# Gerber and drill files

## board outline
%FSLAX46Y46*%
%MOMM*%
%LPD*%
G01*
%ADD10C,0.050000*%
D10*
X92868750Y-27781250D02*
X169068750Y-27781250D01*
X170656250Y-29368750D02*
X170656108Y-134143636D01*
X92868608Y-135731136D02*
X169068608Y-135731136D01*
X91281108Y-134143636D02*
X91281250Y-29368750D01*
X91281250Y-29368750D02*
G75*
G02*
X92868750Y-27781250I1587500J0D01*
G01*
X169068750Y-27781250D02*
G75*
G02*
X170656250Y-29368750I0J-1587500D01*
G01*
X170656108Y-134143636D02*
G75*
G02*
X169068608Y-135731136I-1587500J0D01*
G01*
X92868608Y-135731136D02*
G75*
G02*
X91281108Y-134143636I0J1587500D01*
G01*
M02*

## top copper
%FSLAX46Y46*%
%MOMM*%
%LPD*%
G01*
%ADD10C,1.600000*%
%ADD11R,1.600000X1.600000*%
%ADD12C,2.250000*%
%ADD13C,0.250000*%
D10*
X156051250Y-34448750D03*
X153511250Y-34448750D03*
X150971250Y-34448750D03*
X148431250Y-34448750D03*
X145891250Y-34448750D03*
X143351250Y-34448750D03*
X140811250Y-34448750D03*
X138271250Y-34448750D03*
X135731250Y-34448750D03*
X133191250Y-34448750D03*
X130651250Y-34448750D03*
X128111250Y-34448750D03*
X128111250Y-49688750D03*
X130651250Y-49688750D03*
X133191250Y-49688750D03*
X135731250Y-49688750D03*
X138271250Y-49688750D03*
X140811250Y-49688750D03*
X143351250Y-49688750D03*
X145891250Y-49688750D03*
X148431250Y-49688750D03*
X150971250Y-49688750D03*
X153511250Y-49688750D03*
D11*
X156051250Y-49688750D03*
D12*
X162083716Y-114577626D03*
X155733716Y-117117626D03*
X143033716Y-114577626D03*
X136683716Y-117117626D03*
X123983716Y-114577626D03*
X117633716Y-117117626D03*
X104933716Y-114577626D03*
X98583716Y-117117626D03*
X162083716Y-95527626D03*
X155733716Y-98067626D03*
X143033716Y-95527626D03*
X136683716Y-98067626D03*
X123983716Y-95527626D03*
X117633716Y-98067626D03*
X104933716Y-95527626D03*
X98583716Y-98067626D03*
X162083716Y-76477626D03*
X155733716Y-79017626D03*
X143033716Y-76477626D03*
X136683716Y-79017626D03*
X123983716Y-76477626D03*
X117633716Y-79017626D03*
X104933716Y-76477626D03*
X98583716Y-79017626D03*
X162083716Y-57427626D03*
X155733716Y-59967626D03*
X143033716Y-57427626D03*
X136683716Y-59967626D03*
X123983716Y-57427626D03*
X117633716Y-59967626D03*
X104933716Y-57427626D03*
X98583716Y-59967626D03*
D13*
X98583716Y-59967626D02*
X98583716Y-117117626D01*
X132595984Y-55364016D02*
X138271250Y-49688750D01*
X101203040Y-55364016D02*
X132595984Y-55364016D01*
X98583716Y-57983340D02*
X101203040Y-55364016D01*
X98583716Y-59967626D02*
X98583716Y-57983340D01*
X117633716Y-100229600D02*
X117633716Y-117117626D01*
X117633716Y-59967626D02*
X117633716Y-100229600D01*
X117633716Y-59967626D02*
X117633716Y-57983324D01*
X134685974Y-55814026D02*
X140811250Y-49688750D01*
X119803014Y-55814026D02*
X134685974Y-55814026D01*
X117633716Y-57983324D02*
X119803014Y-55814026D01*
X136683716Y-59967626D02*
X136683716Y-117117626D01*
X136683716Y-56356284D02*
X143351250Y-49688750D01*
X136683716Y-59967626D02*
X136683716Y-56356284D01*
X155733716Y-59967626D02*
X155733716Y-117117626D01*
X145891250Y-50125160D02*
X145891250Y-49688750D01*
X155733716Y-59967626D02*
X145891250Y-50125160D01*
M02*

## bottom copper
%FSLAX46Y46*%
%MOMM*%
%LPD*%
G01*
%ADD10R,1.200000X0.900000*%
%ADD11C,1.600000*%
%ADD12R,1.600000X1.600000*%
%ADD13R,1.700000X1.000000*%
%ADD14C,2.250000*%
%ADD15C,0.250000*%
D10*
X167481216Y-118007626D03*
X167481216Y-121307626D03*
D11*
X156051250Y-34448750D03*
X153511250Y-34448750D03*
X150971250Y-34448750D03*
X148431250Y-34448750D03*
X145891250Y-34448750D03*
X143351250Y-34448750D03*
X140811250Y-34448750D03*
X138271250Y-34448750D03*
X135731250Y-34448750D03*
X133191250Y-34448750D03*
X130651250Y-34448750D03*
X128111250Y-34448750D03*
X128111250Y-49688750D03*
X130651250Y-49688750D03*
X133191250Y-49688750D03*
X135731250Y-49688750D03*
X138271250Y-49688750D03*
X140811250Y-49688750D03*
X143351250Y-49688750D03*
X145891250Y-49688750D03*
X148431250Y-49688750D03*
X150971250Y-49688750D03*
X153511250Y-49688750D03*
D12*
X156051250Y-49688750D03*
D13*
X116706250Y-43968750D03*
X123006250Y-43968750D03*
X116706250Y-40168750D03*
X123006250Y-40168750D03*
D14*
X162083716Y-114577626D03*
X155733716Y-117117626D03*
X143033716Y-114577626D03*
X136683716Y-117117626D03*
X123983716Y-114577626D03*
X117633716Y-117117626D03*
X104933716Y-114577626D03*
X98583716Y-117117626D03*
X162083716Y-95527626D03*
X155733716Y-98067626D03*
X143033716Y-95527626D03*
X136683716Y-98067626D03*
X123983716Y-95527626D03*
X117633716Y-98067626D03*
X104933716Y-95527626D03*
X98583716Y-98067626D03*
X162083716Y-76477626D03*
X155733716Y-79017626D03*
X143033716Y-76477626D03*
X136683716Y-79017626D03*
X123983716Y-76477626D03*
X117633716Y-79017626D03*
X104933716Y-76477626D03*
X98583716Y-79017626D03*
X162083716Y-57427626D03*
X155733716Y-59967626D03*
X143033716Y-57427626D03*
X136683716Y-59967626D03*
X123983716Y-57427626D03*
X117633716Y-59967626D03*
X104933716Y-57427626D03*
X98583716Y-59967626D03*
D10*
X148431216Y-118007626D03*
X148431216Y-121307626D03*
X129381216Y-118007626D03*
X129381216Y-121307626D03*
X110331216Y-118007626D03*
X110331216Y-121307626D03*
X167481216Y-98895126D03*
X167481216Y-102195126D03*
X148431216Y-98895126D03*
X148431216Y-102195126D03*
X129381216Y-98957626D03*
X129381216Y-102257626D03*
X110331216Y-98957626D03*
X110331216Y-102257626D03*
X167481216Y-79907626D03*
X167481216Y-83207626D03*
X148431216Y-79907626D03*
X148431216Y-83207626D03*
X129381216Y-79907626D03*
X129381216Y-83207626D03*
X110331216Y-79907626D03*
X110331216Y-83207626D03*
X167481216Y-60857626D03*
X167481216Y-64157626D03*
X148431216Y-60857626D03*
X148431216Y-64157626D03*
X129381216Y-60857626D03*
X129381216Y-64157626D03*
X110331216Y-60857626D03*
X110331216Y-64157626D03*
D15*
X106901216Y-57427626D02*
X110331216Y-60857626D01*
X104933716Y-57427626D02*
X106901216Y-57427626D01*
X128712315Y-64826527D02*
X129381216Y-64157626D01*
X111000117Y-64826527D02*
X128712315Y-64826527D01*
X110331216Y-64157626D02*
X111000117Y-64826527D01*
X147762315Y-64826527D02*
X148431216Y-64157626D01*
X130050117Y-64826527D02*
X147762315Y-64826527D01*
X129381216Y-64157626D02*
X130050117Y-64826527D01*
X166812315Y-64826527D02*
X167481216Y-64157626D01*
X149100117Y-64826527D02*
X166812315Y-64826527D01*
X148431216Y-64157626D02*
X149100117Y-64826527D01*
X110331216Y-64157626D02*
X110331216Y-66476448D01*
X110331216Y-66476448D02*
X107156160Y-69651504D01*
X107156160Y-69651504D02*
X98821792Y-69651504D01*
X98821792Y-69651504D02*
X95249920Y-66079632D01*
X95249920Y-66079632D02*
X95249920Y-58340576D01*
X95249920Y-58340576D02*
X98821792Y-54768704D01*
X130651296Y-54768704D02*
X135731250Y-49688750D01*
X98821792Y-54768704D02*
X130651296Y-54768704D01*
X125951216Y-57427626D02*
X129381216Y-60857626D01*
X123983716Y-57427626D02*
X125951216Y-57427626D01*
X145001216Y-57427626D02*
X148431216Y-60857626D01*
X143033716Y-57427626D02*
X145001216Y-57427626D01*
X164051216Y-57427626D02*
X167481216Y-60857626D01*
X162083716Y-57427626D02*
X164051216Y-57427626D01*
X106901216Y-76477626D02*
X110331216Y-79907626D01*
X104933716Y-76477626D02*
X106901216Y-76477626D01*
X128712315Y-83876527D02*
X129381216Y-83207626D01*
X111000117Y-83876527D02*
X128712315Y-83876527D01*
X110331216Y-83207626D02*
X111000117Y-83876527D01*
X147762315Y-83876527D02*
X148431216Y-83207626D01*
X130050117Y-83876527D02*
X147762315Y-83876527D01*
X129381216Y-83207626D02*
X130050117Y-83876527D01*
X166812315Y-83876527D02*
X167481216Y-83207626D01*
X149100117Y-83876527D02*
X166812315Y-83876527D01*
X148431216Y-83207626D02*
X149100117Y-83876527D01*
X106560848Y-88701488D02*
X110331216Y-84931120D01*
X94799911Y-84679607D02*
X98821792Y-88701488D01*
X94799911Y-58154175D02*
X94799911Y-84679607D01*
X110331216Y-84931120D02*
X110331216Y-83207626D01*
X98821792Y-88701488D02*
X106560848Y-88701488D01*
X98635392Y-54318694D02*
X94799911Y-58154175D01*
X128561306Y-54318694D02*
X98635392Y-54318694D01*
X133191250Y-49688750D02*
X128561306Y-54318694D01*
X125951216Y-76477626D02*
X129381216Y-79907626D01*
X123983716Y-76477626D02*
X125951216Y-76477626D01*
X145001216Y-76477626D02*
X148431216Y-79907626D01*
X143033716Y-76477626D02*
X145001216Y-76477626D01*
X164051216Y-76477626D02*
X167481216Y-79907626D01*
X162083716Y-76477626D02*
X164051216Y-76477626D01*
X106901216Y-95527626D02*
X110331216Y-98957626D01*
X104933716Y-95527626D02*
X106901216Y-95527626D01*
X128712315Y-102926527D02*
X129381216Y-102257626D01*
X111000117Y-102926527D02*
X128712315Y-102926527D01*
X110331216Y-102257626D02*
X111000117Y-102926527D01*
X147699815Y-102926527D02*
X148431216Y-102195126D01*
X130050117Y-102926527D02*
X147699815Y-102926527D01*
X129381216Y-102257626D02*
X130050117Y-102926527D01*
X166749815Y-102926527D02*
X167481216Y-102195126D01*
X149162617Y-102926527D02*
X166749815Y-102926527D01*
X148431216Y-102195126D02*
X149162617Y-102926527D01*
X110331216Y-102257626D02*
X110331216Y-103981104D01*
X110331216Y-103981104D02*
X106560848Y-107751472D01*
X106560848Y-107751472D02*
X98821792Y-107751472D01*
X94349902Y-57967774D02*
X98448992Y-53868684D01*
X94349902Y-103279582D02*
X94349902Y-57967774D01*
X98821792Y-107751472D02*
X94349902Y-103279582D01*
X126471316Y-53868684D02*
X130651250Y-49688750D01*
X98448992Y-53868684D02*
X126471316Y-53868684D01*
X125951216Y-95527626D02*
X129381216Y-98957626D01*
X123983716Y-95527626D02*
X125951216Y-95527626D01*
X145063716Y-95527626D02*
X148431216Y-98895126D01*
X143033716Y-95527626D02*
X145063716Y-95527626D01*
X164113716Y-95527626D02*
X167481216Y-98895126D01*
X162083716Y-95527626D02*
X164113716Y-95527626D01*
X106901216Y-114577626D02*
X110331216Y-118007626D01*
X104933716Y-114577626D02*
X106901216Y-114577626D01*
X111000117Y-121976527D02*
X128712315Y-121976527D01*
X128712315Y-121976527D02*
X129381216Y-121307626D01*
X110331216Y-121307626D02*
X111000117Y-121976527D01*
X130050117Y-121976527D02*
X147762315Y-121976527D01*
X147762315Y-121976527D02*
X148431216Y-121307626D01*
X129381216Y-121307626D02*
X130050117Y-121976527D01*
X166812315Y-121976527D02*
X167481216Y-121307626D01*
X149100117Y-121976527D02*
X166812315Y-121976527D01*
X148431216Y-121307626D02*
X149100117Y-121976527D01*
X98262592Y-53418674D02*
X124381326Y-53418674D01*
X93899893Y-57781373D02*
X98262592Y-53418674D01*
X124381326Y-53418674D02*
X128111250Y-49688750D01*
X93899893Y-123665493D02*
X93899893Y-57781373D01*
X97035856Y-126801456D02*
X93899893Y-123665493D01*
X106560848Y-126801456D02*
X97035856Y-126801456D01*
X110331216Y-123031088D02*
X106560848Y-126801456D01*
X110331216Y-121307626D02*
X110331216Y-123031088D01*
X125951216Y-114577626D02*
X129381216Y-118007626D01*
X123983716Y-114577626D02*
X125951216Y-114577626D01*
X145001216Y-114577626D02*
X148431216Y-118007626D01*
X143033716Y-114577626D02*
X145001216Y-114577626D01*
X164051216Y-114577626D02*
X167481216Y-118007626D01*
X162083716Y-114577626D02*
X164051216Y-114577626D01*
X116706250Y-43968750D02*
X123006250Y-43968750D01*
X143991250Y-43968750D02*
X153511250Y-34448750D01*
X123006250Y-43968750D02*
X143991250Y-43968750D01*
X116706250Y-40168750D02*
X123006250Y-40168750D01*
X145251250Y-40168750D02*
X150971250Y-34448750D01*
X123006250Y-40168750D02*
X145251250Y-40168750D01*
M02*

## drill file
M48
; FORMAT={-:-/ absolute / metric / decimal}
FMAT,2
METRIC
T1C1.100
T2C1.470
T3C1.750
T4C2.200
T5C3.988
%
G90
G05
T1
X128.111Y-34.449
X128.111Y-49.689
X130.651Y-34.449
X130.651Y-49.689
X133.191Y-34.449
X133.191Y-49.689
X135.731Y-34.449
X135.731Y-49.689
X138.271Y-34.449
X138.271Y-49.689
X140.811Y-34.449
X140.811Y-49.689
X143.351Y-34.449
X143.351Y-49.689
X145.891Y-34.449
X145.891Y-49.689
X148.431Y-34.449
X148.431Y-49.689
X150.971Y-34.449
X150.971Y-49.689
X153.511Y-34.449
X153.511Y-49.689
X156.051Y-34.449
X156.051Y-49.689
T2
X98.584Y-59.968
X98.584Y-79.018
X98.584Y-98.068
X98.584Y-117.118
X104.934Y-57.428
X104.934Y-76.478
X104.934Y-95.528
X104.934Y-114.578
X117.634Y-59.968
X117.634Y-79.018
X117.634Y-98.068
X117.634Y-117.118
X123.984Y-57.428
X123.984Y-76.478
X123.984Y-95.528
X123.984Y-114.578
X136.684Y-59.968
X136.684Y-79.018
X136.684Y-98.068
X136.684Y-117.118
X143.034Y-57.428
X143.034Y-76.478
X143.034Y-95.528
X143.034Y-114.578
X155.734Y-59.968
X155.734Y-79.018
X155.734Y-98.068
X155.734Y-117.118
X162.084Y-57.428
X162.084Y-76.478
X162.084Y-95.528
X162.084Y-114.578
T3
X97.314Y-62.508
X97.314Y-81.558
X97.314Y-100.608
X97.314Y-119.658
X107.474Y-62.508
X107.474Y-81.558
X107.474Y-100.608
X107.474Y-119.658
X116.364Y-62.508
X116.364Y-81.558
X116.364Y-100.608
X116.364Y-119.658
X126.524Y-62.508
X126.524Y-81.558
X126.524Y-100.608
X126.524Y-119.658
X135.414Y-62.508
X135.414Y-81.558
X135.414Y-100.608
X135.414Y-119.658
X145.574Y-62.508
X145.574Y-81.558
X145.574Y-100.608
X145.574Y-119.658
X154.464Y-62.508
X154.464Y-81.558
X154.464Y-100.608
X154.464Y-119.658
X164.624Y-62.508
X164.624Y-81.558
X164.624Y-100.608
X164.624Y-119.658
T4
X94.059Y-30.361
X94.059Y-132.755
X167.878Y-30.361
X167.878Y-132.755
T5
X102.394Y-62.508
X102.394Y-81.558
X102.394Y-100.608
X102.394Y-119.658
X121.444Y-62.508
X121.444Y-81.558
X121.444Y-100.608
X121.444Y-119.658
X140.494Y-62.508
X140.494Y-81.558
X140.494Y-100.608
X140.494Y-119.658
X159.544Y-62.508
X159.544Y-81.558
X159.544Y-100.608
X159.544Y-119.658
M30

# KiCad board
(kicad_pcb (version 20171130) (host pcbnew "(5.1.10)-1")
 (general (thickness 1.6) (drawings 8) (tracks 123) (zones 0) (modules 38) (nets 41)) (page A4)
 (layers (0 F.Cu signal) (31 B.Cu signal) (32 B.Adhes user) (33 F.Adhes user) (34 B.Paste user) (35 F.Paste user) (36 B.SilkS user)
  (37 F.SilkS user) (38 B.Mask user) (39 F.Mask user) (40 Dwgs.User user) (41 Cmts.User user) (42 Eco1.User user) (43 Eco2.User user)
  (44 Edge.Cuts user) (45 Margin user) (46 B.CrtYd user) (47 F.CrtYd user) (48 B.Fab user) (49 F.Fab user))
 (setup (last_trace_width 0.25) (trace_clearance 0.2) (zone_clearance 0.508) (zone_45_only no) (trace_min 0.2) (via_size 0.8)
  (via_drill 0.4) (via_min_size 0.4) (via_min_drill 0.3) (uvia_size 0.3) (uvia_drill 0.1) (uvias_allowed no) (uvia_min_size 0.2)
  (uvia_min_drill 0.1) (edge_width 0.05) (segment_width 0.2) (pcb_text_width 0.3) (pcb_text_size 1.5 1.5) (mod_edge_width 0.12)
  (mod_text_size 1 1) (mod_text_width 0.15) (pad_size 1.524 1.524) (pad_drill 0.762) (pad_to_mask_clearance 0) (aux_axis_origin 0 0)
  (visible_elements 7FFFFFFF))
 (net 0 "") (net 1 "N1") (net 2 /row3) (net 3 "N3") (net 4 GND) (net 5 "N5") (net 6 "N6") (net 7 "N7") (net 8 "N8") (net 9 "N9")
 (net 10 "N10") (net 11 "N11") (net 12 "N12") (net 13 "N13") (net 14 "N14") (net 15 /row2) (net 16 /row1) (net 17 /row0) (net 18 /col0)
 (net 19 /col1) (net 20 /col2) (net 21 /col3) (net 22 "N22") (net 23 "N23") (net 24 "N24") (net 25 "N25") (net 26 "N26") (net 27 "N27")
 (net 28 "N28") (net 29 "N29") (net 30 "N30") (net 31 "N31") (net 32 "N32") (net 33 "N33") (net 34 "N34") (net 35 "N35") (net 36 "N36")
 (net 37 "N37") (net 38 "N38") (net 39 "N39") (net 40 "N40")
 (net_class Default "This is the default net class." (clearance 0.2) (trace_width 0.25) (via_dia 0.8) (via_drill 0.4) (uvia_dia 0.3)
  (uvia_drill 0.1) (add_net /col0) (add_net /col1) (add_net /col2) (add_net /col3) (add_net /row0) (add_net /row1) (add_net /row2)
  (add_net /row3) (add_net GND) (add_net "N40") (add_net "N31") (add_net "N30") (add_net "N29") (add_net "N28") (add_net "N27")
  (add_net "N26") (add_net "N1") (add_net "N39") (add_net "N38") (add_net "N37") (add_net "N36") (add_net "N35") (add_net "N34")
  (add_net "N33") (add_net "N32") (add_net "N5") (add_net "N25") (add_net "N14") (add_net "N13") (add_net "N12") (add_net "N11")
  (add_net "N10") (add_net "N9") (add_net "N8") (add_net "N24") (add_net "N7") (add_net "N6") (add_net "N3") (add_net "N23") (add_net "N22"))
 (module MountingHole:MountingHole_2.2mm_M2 (layer F.Cu) (at 167.877984 132.754576)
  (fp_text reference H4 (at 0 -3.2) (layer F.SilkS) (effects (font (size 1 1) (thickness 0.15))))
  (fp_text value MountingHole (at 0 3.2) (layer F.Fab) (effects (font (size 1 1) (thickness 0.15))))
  (pad 1 np_thru_hole circle (at 0 0) (size 2.2 2.2) (drill 2.2) (layers *.Cu *.Mask)))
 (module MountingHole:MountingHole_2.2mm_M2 (layer F.Cu) (at 94.059296 132.754576)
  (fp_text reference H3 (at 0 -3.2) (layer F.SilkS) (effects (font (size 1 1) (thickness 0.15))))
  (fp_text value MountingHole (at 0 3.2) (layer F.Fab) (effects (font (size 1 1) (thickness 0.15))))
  (pad 1 np_thru_hole circle (at 0 0) (size 2.2 2.2) (drill 2.2) (layers *.Cu *.Mask)))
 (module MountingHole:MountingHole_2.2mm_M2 (layer F.Cu) (at 167.877984 30.360912)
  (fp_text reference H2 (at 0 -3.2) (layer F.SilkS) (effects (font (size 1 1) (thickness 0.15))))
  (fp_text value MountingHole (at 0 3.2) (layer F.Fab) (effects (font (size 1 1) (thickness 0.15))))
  (pad 1 np_thru_hole circle (at 0 0) (size 2.2 2.2) (drill 2.2) (layers *.Cu *.Mask)))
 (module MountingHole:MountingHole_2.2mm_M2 (layer F.Cu) (at 94.059296 30.360912)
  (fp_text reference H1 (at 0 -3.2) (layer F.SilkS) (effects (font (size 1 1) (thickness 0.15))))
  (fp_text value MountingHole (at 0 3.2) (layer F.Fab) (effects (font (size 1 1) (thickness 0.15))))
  (pad 1 np_thru_hole circle (at 0 0) (size 2.2 2.2) (drill 2.2) (layers *.Cu *.Mask)))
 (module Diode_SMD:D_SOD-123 (layer B.Cu) (at 167.481216 119.657626 90)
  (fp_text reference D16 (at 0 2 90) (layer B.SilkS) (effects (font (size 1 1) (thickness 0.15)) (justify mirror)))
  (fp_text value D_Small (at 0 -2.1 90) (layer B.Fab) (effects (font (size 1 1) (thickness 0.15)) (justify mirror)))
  (pad 2 smd rect (at 1.65 0 90) (size 0.9 1.2) (layers B.Cu B.Paste B.Mask) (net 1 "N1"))
  (pad 1 smd rect (at -1.65 0 90) (size 0.9 1.2) (layers B.Cu B.Paste B.Mask) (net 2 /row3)))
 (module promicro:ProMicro (layer B.Cu) (at 142.08125 42.06875 180)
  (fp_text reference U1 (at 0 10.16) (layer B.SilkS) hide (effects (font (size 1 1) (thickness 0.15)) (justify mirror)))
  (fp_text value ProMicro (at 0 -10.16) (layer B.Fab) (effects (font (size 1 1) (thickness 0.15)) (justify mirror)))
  (pad 24 thru_hole circle (at -13.97 7.62 180) (size 1.6 1.6) (drill 1.1) (layers *.Cu *.Mask B.SilkS) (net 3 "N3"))
  (pad 23 thru_hole circle (at -11.43 7.62 180) (size 1.6 1.6) (drill 1.1) (layers *.Cu *.Mask B.SilkS) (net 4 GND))
  (pad 22 thru_hole circle (at -8.89 7.62 180) (size 1.6 1.6) (drill 1.1) (layers *.Cu *.Mask B.SilkS) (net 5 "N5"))
  (pad 21 thru_hole circle (at -6.35 7.62 180) (size 1.6 1.6) (drill 1.1) (layers *.Cu *.Mask B.SilkS) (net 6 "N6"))
  (pad 20 thru_hole circle (at -3.81 7.62 180) (size 1.6 1.6) (drill 1.1) (layers *.Cu *.Mask B.SilkS) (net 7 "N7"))
  (pad 19 thru_hole circle (at -1.27 7.62 180) (size 1.6 1.6) (drill 1.1) (layers *.Cu *.Mask B.SilkS) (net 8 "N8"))
  (pad 18 thru_hole circle (at 1.27 7.62 180) (size 1.6 1.6) (drill 1.1) (layers *.Cu *.Mask B.SilkS) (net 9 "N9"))
  (pad 17 thru_hole circle (at 3.81 7.62 180) (size 1.6 1.6) (drill 1.1) (layers *.Cu *.Mask B.SilkS) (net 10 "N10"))
  (pad 16 thru_hole circle (at 6.35 7.62 180) (size 1.6 1.6) (drill 1.1) (layers *.Cu *.Mask B.SilkS) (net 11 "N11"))
  (pad 15 thru_hole circle (at 8.89 7.62 180) (size 1.6 1.6) (drill 1.1) (layers *.Cu *.Mask B.SilkS) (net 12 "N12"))
  (pad 14 thru_hole circle (at 11.43 7.62 180) (size 1.6 1.6) (drill 1.1) (layers *.Cu *.Mask B.SilkS) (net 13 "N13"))
  (pad 13 thru_hole circle (at 13.97 7.62 180) (size 1.6 1.6) (drill 1.1) (layers *.Cu *.Mask B.SilkS) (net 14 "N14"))
  (pad 12 thru_hole circle (at 13.97 -7.62 180) (size 1.6 1.6) (drill 1.1) (layers *.Cu *.Mask B.SilkS) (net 2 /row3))
  (pad 11 thru_hole circle (at 11.43 -7.62 180) (size 1.6 1.6) (drill 1.1) (layers *.Cu *.Mask B.SilkS) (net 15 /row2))
  (pad 10 thru_hole circle (at 8.89 -7.62 180) (size 1.6 1.6) (drill 1.1) (layers *.Cu *.Mask B.SilkS) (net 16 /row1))
  (pad 9 thru_hole circle (at 6.35 -7.62 180) (size 1.6 1.6) (drill 1.1) (layers *.Cu *.Mask B.SilkS) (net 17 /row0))
  (pad 8 thru_hole circle (at 3.81 -7.62 180) (size 1.6 1.6) (drill 1.1) (layers *.Cu *.Mask B.SilkS) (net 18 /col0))
  (pad 7 thru_hole circle (at 1.27 -7.62 180) (size 1.6 1.6) (drill 1.1) (layers *.Cu *.Mask B.SilkS) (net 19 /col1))
  (pad 6 thru_hole circle (at -1.27 -7.62 180) (size 1.6 1.6) (drill 1.1) (layers *.Cu *.Mask B.SilkS) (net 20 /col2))
  (pad 5 thru_hole circle (at -3.81 -7.62 180) (size 1.6 1.6) (drill 1.1) (layers *.Cu *.Mask B.SilkS) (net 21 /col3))
  (pad 4 thru_hole circle (at -6.35 -7.62 180) (size 1.6 1.6) (drill 1.1) (layers *.Cu *.Mask B.SilkS) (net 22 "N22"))
  (pad 3 thru_hole circle (at -8.89 -7.62 180) (size 1.6 1.6) (drill 1.1) (layers *.Cu *.Mask B.SilkS) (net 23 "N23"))
  (pad 2 thru_hole circle (at -11.43 -7.62 180) (size 1.6 1.6) (drill 1.1) (layers *.Cu *.Mask B.SilkS) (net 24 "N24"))
  (pad 1 thru_hole rect (at -13.97 -7.62 180) (size 1.6 1.6) (drill 1.1) (layers *.Cu *.Mask B.SilkS) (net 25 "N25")))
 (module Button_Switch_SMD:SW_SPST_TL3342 (layer B.Cu) (at 119.85625 42.06875 180)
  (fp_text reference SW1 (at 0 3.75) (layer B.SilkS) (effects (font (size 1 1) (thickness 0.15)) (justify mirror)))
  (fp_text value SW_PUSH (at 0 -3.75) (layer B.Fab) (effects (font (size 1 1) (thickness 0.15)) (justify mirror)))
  (pad 2 smd rect (at 3.15 -1.9 180) (size 1.7 1) (layers B.Cu B.Paste B.Mask) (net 4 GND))
  (pad 2 smd rect (at -3.15 -1.9 180) (size 1.7 1) (layers B.Cu B.Paste B.Mask) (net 4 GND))
  (pad 1 smd rect (at 3.15 1.9 180) (size 1.7 1) (layers B.Cu B.Paste B.Mask) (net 5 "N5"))
  (pad 1 smd rect (at -3.15 1.9 180) (size 1.7 1) (layers B.Cu B.Paste B.Mask) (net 5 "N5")))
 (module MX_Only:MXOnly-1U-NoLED (layer F.Cu) (at 159.543716 119.657626)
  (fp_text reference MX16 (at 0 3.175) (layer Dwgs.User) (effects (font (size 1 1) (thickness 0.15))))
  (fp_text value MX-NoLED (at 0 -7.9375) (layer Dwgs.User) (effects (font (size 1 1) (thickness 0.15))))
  (pad 2 thru_hole circle (at 2.54 -5.08) (size 2.25 2.25) (drill 1.47) (layers *.Cu B.Mask) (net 1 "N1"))
  (pad "" np_thru_hole circle (at 0 0) (size 3.9878 3.9878) (drill 3.9878) (layers *.Cu *.Mask))
  (pad 1 thru_hole circle (at -3.81 -2.54) (size 2.25 2.25) (drill 1.47) (layers *.Cu B.Mask) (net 21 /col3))
  (pad "" np_thru_hole circle (at -5.08 0 48.0996) (size 1.75 1.75) (drill 1.75) (layers *.Cu *.Mask))
  (pad "" np_thru_hole circle (at 5.08 0 48.0996) (size 1.75 1.75) (drill 1.75) (layers *.Cu *.Mask)))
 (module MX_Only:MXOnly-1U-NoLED (layer F.Cu) (at 140.493716 119.657626)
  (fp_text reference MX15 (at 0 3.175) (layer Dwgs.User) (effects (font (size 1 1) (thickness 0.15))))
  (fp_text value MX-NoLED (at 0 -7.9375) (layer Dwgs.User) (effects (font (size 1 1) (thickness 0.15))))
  (pad 2 thru_hole circle (at 2.54 -5.08) (size 2.25 2.25) (drill 1.47) (layers *.Cu B.Mask) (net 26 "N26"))
  (pad "" np_thru_hole circle (at 0 0) (size 3.9878 3.9878) (drill 3.9878) (layers *.Cu *.Mask))
  (pad 1 thru_hole circle (at -3.81 -2.54) (size 2.25 2.25) (drill 1.47) (layers *.Cu B.Mask) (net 20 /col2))
  (pad "" np_thru_hole circle (at -5.08 0 48.0996) (size 1.75 1.75) (drill 1.75) (layers *.Cu *.Mask))
  (pad "" np_thru_hole circle (at 5.08 0 48.0996) (size 1.75 1.75) (drill 1.75) (layers *.Cu *.Mask)))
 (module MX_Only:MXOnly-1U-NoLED (layer F.Cu) (at 121.443716 119.657626)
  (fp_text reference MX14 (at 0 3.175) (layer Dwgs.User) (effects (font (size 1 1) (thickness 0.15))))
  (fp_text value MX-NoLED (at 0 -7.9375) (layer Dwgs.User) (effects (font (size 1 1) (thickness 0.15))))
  (pad 2 thru_hole circle (at 2.54 -5.08) (size 2.25 2.25) (drill 1.47) (layers *.Cu B.Mask) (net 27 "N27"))
  (pad "" np_thru_hole circle (at 0 0) (size 3.9878 3.9878) (drill 3.9878) (layers *.Cu *.Mask))
  (pad 1 thru_hole circle (at -3.81 -2.54) (size 2.25 2.25) (drill 1.47) (layers *.Cu B.Mask) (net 19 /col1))
  (pad "" np_thru_hole circle (at -5.08 0 48.0996) (size 1.75 1.75) (drill 1.75) (layers *.Cu *.Mask))
  (pad "" np_thru_hole circle (at 5.08 0 48.0996) (size 1.75 1.75) (drill 1.75) (layers *.Cu *.Mask)))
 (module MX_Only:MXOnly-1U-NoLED (layer F.Cu) (at 102.393716 119.657626)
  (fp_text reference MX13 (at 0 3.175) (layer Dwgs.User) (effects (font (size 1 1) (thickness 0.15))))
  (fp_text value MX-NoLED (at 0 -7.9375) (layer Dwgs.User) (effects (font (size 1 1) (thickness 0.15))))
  (pad 2 thru_hole circle (at 2.54 -5.08) (size 2.25 2.25) (drill 1.47) (layers *.Cu B.Mask) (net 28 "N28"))
  (pad "" np_thru_hole circle (at 0 0) (size 3.9878 3.9878) (drill 3.9878) (layers *.Cu *.Mask))
  (pad 1 thru_hole circle (at -3.81 -2.54) (size 2.25 2.25) (drill 1.47) (layers *.Cu B.Mask) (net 18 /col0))
  (pad "" np_thru_hole circle (at -5.08 0 48.0996) (size 1.75 1.75) (drill 1.75) (layers *.Cu *.Mask))
  (pad "" np_thru_hole circle (at 5.08 0 48.0996) (size 1.75 1.75) (drill 1.75) (layers *.Cu *.Mask)))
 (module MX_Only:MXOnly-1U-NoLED (layer F.Cu) (at 159.543716 100.607626)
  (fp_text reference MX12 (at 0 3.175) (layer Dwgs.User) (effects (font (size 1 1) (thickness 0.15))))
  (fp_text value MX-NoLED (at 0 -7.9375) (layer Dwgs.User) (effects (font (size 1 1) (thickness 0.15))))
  (pad 2 thru_hole circle (at 2.54 -5.08) (size 2.25 2.25) (drill 1.47) (layers *.Cu B.Mask) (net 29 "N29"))
  (pad "" np_thru_hole circle (at 0 0) (size 3.9878 3.9878) (drill 3.9878) (layers *.Cu *.Mask))
  (pad 1 thru_hole circle (at -3.81 -2.54) (size 2.25 2.25) (drill 1.47) (layers *.Cu B.Mask) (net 21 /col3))
  (pad "" np_thru_hole circle (at -5.08 0 48.0996) (size 1.75 1.75) (drill 1.75) (layers *.Cu *.Mask))
  (pad "" np_thru_hole circle (at 5.08 0 48.0996) (size 1.75 1.75) (drill 1.75) (layers *.Cu *.Mask)))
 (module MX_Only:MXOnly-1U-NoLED (layer F.Cu) (at 140.493716 100.607626)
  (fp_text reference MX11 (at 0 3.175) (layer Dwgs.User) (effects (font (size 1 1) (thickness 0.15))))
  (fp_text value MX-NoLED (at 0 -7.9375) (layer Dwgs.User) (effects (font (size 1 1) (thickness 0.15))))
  (pad 2 thru_hole circle (at 2.54 -5.08) (size 2.25 2.25) (drill 1.47) (layers *.Cu B.Mask) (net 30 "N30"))
  (pad "" np_thru_hole circle (at 0 0) (size 3.9878 3.9878) (drill 3.9878) (layers *.Cu *.Mask))
  (pad 1 thru_hole circle (at -3.81 -2.54) (size 2.25 2.25) (drill 1.47) (layers *.Cu B.Mask) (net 20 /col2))
  (pad "" np_thru_hole circle (at -5.08 0 48.0996) (size 1.75 1.75) (drill 1.75) (layers *.Cu *.Mask))
  (pad "" np_thru_hole circle (at 5.08 0 48.0996) (size 1.75 1.75) (drill 1.75) (layers *.Cu *.Mask)))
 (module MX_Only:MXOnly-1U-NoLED (layer F.Cu) (at 121.443716 100.607626)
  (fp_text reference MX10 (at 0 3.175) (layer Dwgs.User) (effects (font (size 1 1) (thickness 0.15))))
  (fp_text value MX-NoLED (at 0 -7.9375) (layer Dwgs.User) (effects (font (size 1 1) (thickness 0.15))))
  (pad 2 thru_hole circle (at 2.54 -5.08) (size 2.25 2.25) (drill 1.47) (layers *.Cu B.Mask) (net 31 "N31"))
  (pad "" np_thru_hole circle (at 0 0) (size 3.9878 3.9878) (drill 3.9878) (layers *.Cu *.Mask))
  (pad 1 thru_hole circle (at -3.81 -2.54) (size 2.25 2.25) (drill 1.47) (layers *.Cu B.Mask) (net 19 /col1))
  (pad "" np_thru_hole circle (at -5.08 0 48.0996) (size 1.75 1.75) (drill 1.75) (layers *.Cu *.Mask))
  (pad "" np_thru_hole circle (at 5.08 0 48.0996) (size 1.75 1.75) (drill 1.75) (layers *.Cu *.Mask)))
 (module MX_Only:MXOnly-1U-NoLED (layer F.Cu) (at 102.393716 100.607626)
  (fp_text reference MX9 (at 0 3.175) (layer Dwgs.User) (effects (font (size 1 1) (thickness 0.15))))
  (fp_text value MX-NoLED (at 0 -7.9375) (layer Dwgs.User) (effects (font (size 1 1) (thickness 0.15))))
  (pad 2 thru_hole circle (at 2.54 -5.08) (size 2.25 2.25) (drill 1.47) (layers *.Cu B.Mask) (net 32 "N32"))
  (pad "" np_thru_hole circle (at 0 0) (size 3.9878 3.9878) (drill 3.9878) (layers *.Cu *.Mask))
  (pad 1 thru_hole circle (at -3.81 -2.54) (size 2.25 2.25) (drill 1.47) (layers *.Cu B.Mask) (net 18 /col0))
  (pad "" np_thru_hole circle (at -5.08 0 48.0996) (size 1.75 1.75) (drill 1.75) (layers *.Cu *.Mask))
  (pad "" np_thru_hole circle (at 5.08 0 48.0996) (size 1.75 1.75) (drill 1.75) (layers *.Cu *.Mask)))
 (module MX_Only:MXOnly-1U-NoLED (layer F.Cu) (at 159.543716 81.557626)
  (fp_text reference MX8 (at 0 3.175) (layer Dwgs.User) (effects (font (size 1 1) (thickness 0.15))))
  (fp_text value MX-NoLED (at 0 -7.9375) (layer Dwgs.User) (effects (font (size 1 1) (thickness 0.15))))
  (pad 2 thru_hole circle (at 2.54 -5.08) (size 2.25 2.25) (drill 1.47) (layers *.Cu B.Mask) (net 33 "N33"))
  (pad "" np_thru_hole circle (at 0 0) (size 3.9878 3.9878) (drill 3.9878) (layers *.Cu *.Mask))
  (pad 1 thru_hole circle (at -3.81 -2.54) (size 2.25 2.25) (drill 1.47) (layers *.Cu B.Mask) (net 21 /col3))
  (pad "" np_thru_hole circle (at -5.08 0 48.0996) (size 1.75 1.75) (drill 1.75) (layers *.Cu *.Mask))
  (pad "" np_thru_hole circle (at 5.08 0 48.0996) (size 1.75 1.75) (drill 1.75) (layers *.Cu *.Mask)))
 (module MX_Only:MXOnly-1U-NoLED (layer F.Cu) (at 140.493716 81.557626)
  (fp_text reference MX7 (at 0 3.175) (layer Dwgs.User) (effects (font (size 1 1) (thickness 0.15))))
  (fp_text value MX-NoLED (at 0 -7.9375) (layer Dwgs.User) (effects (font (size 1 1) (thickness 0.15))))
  (pad 2 thru_hole circle (at 2.54 -5.08) (size 2.25 2.25) (drill 1.47) (layers *.Cu B.Mask) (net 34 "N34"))
  (pad "" np_thru_hole circle (at 0 0) (size 3.9878 3.9878) (drill 3.9878) (layers *.Cu *.Mask))
  (pad 1 thru_hole circle (at -3.81 -2.54) (size 2.25 2.25) (drill 1.47) (layers *.Cu B.Mask) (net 20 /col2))
  (pad "" np_thru_hole circle (at -5.08 0 48.0996) (size 1.75 1.75) (drill 1.75) (layers *.Cu *.Mask))
  (pad "" np_thru_hole circle (at 5.08 0 48.0996) (size 1.75 1.75) (drill 1.75) (layers *.Cu *.Mask)))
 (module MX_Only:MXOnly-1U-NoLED (layer F.Cu) (at 121.443716 81.557626)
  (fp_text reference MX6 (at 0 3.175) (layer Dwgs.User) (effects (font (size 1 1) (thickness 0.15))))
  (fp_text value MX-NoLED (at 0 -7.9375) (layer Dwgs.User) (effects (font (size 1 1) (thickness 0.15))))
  (pad 2 thru_hole circle (at 2.54 -5.08) (size 2.25 2.25) (drill 1.47) (layers *.Cu B.Mask) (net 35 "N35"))
  (pad "" np_thru_hole circle (at 0 0) (size 3.9878 3.9878) (drill 3.9878) (layers *.Cu *.Mask))
  (pad 1 thru_hole circle (at -3.81 -2.54) (size 2.25 2.25) (drill 1.47) (layers *.Cu B.Mask) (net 19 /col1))
  (pad "" np_thru_hole circle (at -5.08 0 48.0996) (size 1.75 1.75) (drill 1.75) (layers *.Cu *.Mask))
  (pad "" np_thru_hole circle (at 5.08 0 48.0996) (size 1.75 1.75) (drill 1.75) (layers *.Cu *.Mask)))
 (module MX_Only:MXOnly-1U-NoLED (layer F.Cu) (at 102.393716 81.557626)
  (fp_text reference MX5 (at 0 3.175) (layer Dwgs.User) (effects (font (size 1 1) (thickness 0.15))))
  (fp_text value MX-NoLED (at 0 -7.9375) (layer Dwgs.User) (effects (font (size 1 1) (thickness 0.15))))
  (pad 2 thru_hole circle (at 2.54 -5.08) (size 2.25 2.25) (drill 1.47) (layers *.Cu B.Mask) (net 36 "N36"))
  (pad "" np_thru_hole circle (at 0 0) (size 3.9878 3.9878) (drill 3.9878) (layers *.Cu *.Mask))
  (pad 1 thru_hole circle (at -3.81 -2.54) (size 2.25 2.25) (drill 1.47) (layers *.Cu B.Mask) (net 18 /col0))
  (pad "" np_thru_hole circle (at -5.08 0 48.0996) (size 1.75 1.75) (drill 1.75) (layers *.Cu *.Mask))
  (pad "" np_thru_hole circle (at 5.08 0 48.0996) (size 1.75 1.75) (drill 1.75) (layers *.Cu *.Mask)))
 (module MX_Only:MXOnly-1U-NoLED (layer F.Cu) (at 159.543716 62.507626)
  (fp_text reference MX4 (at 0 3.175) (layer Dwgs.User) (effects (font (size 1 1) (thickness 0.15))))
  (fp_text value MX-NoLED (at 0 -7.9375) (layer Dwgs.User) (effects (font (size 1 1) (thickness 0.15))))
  (pad 2 thru_hole circle (at 2.54 -5.08) (size 2.25 2.25) (drill 1.47) (layers *.Cu B.Mask) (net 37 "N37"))
  (pad "" np_thru_hole circle (at 0 0) (size 3.9878 3.9878) (drill 3.9878) (layers *.Cu *.Mask))
  (pad 1 thru_hole circle (at -3.81 -2.54) (size 2.25 2.25) (drill 1.47) (layers *.Cu B.Mask) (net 21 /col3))
  (pad "" np_thru_hole circle (at -5.08 0 48.0996) (size 1.75 1.75) (drill 1.75) (layers *.Cu *.Mask))
  (pad "" np_thru_hole circle (at 5.08 0 48.0996) (size 1.75 1.75) (drill 1.75) (layers *.Cu *.Mask)))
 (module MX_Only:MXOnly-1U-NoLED (layer F.Cu) (at 140.493716 62.507626)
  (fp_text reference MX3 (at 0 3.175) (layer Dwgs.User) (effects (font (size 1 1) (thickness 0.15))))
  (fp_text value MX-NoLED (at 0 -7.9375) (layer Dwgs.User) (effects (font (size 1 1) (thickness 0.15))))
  (pad 2 thru_hole circle (at 2.54 -5.08) (size 2.25 2.25) (drill 1.47) (layers *.Cu B.Mask) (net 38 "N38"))
  (pad "" np_thru_hole circle (at 0 0) (size 3.9878 3.9878) (drill 3.9878) (layers *.Cu *.Mask))
  (pad 1 thru_hole circle (at -3.81 -2.54) (size 2.25 2.25) (drill 1.47) (layers *.Cu B.Mask) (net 20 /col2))
  (pad "" np_thru_hole circle (at -5.08 0 48.0996) (size 1.75 1.75) (drill 1.75) (layers *.Cu *.Mask))
  (pad "" np_thru_hole circle (at 5.08 0 48.0996) (size 1.75 1.75) (drill 1.75) (layers *.Cu *.Mask)))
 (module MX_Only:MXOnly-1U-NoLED (layer F.Cu) (at 121.443716 62.507626)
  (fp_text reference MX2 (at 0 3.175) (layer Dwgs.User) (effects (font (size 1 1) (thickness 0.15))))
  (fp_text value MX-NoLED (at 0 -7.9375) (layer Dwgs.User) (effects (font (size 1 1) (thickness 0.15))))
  (pad 2 thru_hole circle (at 2.54 -5.08) (size 2.25 2.25) (drill 1.47) (layers *.Cu B.Mask) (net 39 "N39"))
  (pad "" np_thru_hole circle (at 0 0) (size 3.9878 3.9878) (drill 3.9878) (layers *.Cu *.Mask))
  (pad 1 thru_hole circle (at -3.81 -2.54) (size 2.25 2.25) (drill 1.47) (layers *.Cu B.Mask) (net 19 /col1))
  (pad "" np_thru_hole circle (at -5.08 0 48.0996) (size 1.75 1.75) (drill 1.75) (layers *.Cu *.Mask))
  (pad "" np_thru_hole circle (at 5.08 0 48.0996) (size 1.75 1.75) (drill 1.75) (layers *.Cu *.Mask)))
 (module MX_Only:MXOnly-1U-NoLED (layer F.Cu) (at 102.393716 62.507626)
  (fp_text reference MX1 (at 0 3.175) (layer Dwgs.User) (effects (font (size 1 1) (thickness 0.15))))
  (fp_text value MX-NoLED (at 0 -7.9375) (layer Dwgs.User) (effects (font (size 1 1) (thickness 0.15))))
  (pad 2 thru_hole circle (at 2.54 -5.08) (size 2.25 2.25) (drill 1.47) (layers *.Cu B.Mask) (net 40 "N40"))
  (pad "" np_thru_hole circle (at 0 0) (size 3.9878 3.9878) (drill 3.9878) (layers *.Cu *.Mask))
  (pad 1 thru_hole circle (at -3.81 -2.54) (size 2.25 2.25) (drill 1.47) (layers *.Cu B.Mask) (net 18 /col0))
  (pad "" np_thru_hole circle (at -5.08 0 48.0996) (size 1.75 1.75) (drill 1.75) (layers *.Cu *.Mask))
  (pad "" np_thru_hole circle (at 5.08 0 48.0996) (size 1.75 1.75) (drill 1.75) (layers *.Cu *.Mask)))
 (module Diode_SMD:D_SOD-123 (layer B.Cu) (at 148.431216 119.657626 90)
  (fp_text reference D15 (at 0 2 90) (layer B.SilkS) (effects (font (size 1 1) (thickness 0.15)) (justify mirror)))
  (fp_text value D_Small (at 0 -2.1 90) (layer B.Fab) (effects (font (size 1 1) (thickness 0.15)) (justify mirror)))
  (pad 2 smd rect (at 1.65 0 90) (size 0.9 1.2) (layers B.Cu B.Paste B.Mask) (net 26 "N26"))
  (pad 1 smd rect (at -1.65 0 90) (size 0.9 1.2) (layers B.Cu B.Paste B.Mask) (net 2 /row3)))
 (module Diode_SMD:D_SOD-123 (layer B.Cu) (at 129.381216 119.657626 90)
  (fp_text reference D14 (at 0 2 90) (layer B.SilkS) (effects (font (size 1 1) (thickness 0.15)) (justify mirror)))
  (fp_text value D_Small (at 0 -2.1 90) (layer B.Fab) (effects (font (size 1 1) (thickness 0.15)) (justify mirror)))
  (pad 2 smd rect (at 1.65 0 90) (size 0.9 1.2) (layers B.Cu B.Paste B.Mask) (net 27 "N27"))
  (pad 1 smd rect (at -1.65 0 90) (size 0.9 1.2) (layers B.Cu B.Paste B.Mask) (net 2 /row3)))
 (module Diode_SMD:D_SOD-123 (layer B.Cu) (at 110.331216 119.657626 90)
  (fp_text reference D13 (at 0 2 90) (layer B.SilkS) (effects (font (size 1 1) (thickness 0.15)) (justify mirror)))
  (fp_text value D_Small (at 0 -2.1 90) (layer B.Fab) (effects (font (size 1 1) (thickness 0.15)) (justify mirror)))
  (pad 2 smd rect (at 1.65 0 90) (size 0.9 1.2) (layers B.Cu B.Paste B.Mask) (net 28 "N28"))
  (pad 1 smd rect (at -1.65 0 90) (size 0.9 1.2) (layers B.Cu B.Paste B.Mask) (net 2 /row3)))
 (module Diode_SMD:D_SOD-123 (layer B.Cu) (at 167.481216 100.545126 90)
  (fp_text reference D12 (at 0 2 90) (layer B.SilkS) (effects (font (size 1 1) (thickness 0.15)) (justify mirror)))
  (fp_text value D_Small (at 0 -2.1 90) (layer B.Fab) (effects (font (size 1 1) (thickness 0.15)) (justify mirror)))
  (pad 2 smd rect (at 1.65 0 90) (size 0.9 1.2) (layers B.Cu B.Paste B.Mask) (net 29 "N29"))
  (pad 1 smd rect (at -1.65 0 90) (size 0.9 1.2) (layers B.Cu B.Paste B.Mask) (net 15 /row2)))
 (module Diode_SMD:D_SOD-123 (layer B.Cu) (at 148.431216 100.545126 90)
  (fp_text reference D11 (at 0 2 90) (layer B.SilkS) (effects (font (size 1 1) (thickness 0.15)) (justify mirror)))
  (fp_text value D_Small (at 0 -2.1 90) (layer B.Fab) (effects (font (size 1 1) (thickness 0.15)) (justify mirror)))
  (pad 2 smd rect (at 1.65 0 90) (size 0.9 1.2) (layers B.Cu B.Paste B.Mask) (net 30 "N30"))
  (pad 1 smd rect (at -1.65 0 90) (size 0.9 1.2) (layers B.Cu B.Paste B.Mask) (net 15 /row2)))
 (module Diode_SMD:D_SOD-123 (layer B.Cu) (at 129.381216 100.607626 90)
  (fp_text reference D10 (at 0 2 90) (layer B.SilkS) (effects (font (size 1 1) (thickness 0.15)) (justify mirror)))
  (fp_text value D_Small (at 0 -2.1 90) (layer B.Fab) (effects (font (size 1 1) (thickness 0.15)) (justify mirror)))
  (pad 2 smd rect (at 1.65 0 90) (size 0.9 1.2) (layers B.Cu B.Paste B.Mask) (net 31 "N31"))
  (pad 1 smd rect (at -1.65 0 90) (size 0.9 1.2) (layers B.Cu B.Paste B.Mask) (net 15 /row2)))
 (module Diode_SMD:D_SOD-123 (layer B.Cu) (at 110.331216 100.607626 90)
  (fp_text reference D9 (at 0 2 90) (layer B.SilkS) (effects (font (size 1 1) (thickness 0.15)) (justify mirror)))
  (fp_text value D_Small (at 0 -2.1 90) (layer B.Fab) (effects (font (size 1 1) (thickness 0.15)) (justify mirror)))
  (pad 2 smd rect (at 1.65 0 90) (size 0.9 1.2) (layers B.Cu B.Paste B.Mask) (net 32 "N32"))
  (pad 1 smd rect (at -1.65 0 90) (size 0.9 1.2) (layers B.Cu B.Paste B.Mask) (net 15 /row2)))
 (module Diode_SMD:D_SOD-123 (layer B.Cu) (at 167.481216 81.557626 90)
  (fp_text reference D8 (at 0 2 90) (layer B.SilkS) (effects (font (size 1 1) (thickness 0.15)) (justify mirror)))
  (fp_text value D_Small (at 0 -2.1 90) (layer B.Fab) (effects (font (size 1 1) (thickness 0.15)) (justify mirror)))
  (pad 2 smd rect (at 1.65 0 90) (size 0.9 1.2) (layers B.Cu B.Paste B.Mask) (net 33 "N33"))
  (pad 1 smd rect (at -1.65 0 90) (size 0.9 1.2) (layers B.Cu B.Paste B.Mask) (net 16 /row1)))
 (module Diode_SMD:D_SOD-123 (layer B.Cu) (at 148.431216 81.557626 90)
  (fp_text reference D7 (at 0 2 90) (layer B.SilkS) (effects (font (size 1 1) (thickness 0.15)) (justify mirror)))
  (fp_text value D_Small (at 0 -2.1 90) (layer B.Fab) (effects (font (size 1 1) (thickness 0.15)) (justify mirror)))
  (pad 2 smd rect (at 1.65 0 90) (size 0.9 1.2) (layers B.Cu B.Paste B.Mask) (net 34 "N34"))
  (pad 1 smd rect (at -1.65 0 90) (size 0.9 1.2) (layers B.Cu B.Paste B.Mask) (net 16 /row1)))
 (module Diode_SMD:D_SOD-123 (layer B.Cu) (at 129.381216 81.557626 90)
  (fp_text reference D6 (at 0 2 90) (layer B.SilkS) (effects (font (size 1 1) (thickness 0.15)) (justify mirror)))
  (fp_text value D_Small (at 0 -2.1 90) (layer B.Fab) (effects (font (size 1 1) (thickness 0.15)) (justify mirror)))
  (pad 2 smd rect (at 1.65 0 90) (size 0.9 1.2) (layers B.Cu B.Paste B.Mask) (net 35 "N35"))
  (pad 1 smd rect (at -1.65 0 90) (size 0.9 1.2) (layers B.Cu B.Paste B.Mask) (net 16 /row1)))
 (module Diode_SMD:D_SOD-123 (layer B.Cu) (at 110.331216 81.557626 90)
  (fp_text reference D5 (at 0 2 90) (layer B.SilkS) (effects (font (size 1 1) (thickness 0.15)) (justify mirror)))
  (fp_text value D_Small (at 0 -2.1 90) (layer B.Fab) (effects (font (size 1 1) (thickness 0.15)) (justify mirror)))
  (pad 2 smd rect (at 1.65 0 90) (size 0.9 1.2) (layers B.Cu B.Paste B.Mask) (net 36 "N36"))
  (pad 1 smd rect (at -1.65 0 90) (size 0.9 1.2) (layers B.Cu B.Paste B.Mask) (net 16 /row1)))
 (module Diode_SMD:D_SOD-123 (layer B.Cu) (at 167.481216 62.507626 90)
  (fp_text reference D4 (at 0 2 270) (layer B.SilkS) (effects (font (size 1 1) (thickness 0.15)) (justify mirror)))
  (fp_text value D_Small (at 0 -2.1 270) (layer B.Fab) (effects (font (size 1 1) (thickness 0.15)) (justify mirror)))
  (pad 2 smd rect (at 1.65 0 90) (size 0.9 1.2) (layers B.Cu B.Paste B.Mask) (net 37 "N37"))
  (pad 1 smd rect (at -1.65 0 90) (size 0.9 1.2) (layers B.Cu B.Paste B.Mask) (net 17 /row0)))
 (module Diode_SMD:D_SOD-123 (layer B.Cu) (at 148.431216 62.507626 90)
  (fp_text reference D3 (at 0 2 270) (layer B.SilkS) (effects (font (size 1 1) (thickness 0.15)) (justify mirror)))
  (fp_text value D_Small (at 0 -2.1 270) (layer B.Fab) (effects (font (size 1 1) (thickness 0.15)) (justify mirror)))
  (pad 2 smd rect (at 1.65 0 90) (size 0.9 1.2) (layers B.Cu B.Paste B.Mask) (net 38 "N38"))
  (pad 1 smd rect (at -1.65 0 90) (size 0.9 1.2) (layers B.Cu B.Paste B.Mask) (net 17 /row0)))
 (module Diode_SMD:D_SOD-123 (layer B.Cu) (at 129.381216 62.507626 90)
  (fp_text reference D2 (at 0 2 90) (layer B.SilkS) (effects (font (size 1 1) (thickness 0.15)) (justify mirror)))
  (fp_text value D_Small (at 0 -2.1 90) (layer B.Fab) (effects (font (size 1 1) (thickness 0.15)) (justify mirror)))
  (pad 2 smd rect (at 1.65 0 90) (size 0.9 1.2) (layers B.Cu B.Paste B.Mask) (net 39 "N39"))
  (pad 1 smd rect (at -1.65 0 90) (size 0.9 1.2) (layers B.Cu B.Paste B.Mask) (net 17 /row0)))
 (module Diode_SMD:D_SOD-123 (layer B.Cu) (at 110.331216 62.507626 90)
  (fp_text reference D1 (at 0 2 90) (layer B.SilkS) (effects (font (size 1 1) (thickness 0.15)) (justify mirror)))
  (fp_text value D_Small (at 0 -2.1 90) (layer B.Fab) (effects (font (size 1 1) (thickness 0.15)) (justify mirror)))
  (pad 2 smd rect (at 1.65 0 90) (size 0.9 1.2) (layers B.Cu B.Paste B.Mask) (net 40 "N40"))
  (pad 1 smd rect (at -1.65 0 90) (size 0.9 1.2) (layers B.Cu B.Paste B.Mask) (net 17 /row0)))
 (gr_line (start 92.86875 27.78125) (end 169.06875 27.78125) (layer Edge.Cuts) (width 0.05))
 (gr_line (start 170.65625 29.36875) (end 170.656108 134.143636) (layer Edge.Cuts) (width 0.05))
 (gr_line (start 92.868608 135.731136) (end 169.068608 135.731136) (layer Edge.Cuts) (width 0.05))
 (gr_line (start 91.281108 134.143636) (end 91.28125 29.36875) (layer Edge.Cuts) (width 0.05))
 (gr_arc (start 92.86875 29.36875) (end 92.86875 27.78125) (angle -90) (layer Edge.Cuts) (width 0.05))
 (gr_arc (start 169.06875 29.36875) (end 170.65625 29.36875) (angle -90) (layer Edge.Cuts) (width 0.05))
 (gr_arc (start 169.068608 134.143636) (end 169.068608 135.731136) (angle -90) (layer Edge.Cuts) (width 0.05))
 (gr_arc (start 92.868608 134.143636) (end 91.281108 134.143636) (angle -90) (layer Edge.Cuts) (width 0.05))
 (segment (start 106.901216 57.427626) (end 110.331216 60.857626) (width 0.25) (layer B.Cu) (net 40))
 (segment (start 104.933716 57.427626) (end 106.901216 57.427626) (width 0.25) (layer B.Cu) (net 40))
 (segment (start 128.712315 64.826527) (end 129.381216 64.157626) (width 0.25) (layer B.Cu) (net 17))
 (segment (start 111.000117 64.826527) (end 128.712315 64.826527) (width 0.25) (layer B.Cu) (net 17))
 (segment (start 110.331216 64.157626) (end 111.000117 64.826527) (width 0.25) (layer B.Cu) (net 17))
 (segment (start 147.762315 64.826527) (end 148.431216 64.157626) (width 0.25) (layer B.Cu) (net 17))
 (segment (start 130.050117 64.826527) (end 147.762315 64.826527) (width 0.25) (layer B.Cu) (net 17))
 (segment (start 129.381216 64.157626) (end 130.050117 64.826527) (width 0.25) (layer B.Cu) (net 17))
 (segment (start 166.812315 64.826527) (end 167.481216 64.157626) (width 0.25) (layer B.Cu) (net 17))
 (segment (start 149.100117 64.826527) (end 166.812315 64.826527) (width 0.25) (layer B.Cu) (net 17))
 (segment (start 148.431216 64.157626) (end 149.100117 64.826527) (width 0.25) (layer B.Cu) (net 17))
 (segment (start 110.331216 64.157626) (end 110.331216 66.476448) (width 0.25) (layer B.Cu) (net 17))
 (segment (start 110.331216 66.476448) (end 107.15616 69.651504) (width 0.25) (layer B.Cu) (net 17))
 (segment (start 107.15616 69.651504) (end 98.821792 69.651504) (width 0.25) (layer B.Cu) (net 17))
 (segment (start 98.821792 69.651504) (end 95.24992 66.079632) (width 0.25) (layer B.Cu) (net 17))
 (segment (start 95.24992 66.079632) (end 95.24992 58.340576) (width 0.25) (layer B.Cu) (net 17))
 (segment (start 95.24992 58.340576) (end 98.821792 54.768704) (width 0.25) (layer B.Cu) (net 17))
 (segment (start 130.651296 54.768704) (end 135.73125 49.68875) (width 0.25) (layer B.Cu) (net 17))
 (segment (start 98.821792 54.768704) (end 130.651296 54.768704) (width 0.25) (layer B.Cu) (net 17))
 (segment (start 125.951216 57.427626) (end 129.381216 60.857626) (width 0.25) (layer B.Cu) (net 39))
 (segment (start 123.983716 57.427626) (end 125.951216 57.427626) (width 0.25) (layer B.Cu) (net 39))
 (segment (start 145.001216 57.427626) (end 148.431216 60.857626) (width 0.25) (layer B.Cu) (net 38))
 (segment (start 143.033716 57.427626) (end 145.001216 57.427626) (width 0.25) (layer B.Cu) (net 38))
 (segment (start 164.051216 57.427626) (end 167.481216 60.857626) (width 0.25) (layer B.Cu) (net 37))
 (segment (start 162.083716 57.427626) (end 164.051216 57.427626) (width 0.25) (layer B.Cu) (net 37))
 (segment (start 106.901216 76.477626) (end 110.331216 79.907626) (width 0.25) (layer B.Cu) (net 36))
 (segment (start 104.933716 76.477626) (end 106.901216 76.477626) (width 0.25) (layer B.Cu) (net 36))
 (segment (start 128.712315 83.876527) (end 129.381216 83.207626) (width 0.25) (layer B.Cu) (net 16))
 (segment (start 111.000117 83.876527) (end 128.712315 83.876527) (width 0.25) (layer B.Cu) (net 16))
 (segment (start 110.331216 83.207626) (end 111.000117 83.876527) (width 0.25) (layer B.Cu) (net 16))
 (segment (start 147.762315 83.876527) (end 148.431216 83.207626) (width 0.25) (layer B.Cu) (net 16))
 (segment (start 130.050117 83.876527) (end 147.762315 83.876527) (width 0.25) (layer B.Cu) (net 16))
 (segment (start 129.381216 83.207626) (end 130.050117 83.876527) (width 0.25) (layer B.Cu) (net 16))
 (segment (start 166.812315 83.876527) (end 167.481216 83.207626) (width 0.25) (layer B.Cu) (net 16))
 (segment (start 149.100117 83.876527) (end 166.812315 83.876527) (width 0.25) (layer B.Cu) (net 16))
 (segment (start 148.431216 83.207626) (end 149.100117 83.876527) (width 0.25) (layer B.Cu) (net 16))
 (segment (start 106.560848 88.701488) (end 110.331216 84.93112) (width 0.25) (layer B.Cu) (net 16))
 (segment (start 94.799911 84.679607) (end 98.821792 88.701488) (width 0.25) (layer B.Cu) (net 16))
 (segment (start 94.799911 58.154175) (end 94.799911 84.679607) (width 0.25) (layer B.Cu) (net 16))
 (segment (start 110.331216 84.93112) (end 110.331216 83.207626) (width 0.25) (layer B.Cu) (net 16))
 (segment (start 98.821792 88.701488) (end 106.560848 88.701488) (width 0.25) (layer B.Cu) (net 16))
 (segment (start 98.635392 54.318694) (end 94.799911 58.154175) (width 0.25) (layer B.Cu) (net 16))
 (segment (start 128.561306 54.318694) (end 98.635392 54.318694) (width 0.25) (layer B.Cu) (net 16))
 (segment (start 133.19125 49.68875) (end 128.561306 54.318694) (width 0.25) (layer B.Cu) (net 16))
 (segment (start 125.951216 76.477626) (end 129.381216 79.907626) (width 0.25) (layer B.Cu) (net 35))
 (segment (start 123.983716 76.477626) (end 125.951216 76.477626) (width 0.25) (layer B.Cu) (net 35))
 (segment (start 145.001216 76.477626) (end 148.431216 79.907626) (width 0.25) (layer B.Cu) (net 34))
 (segment (start 143.033716 76.477626) (end 145.001216 76.477626) (width 0.25) (layer B.Cu) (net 34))
 (segment (start 164.051216 76.477626) (end 167.481216 79.907626) (width 0.25) (layer B.Cu) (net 33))
 (segment (start 162.083716 76.477626) (end 164.051216 76.477626) (width 0.25) (layer B.Cu) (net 33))
 (segment (start 106.901216 95.527626) (end 110.331216 98.957626) (width 0.25) (layer B.Cu) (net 32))
 (segment (start 104.933716 95.527626) (end 106.901216 95.527626) (width 0.25) (layer B.Cu) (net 32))
 (segment (start 128.712315 102.926527) (end 129.381216 102.257626) (width 0.25) (layer B.Cu) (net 15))
 (segment (start 111.000117 102.926527) (end 128.712315 102.926527) (width 0.25) (layer B.Cu) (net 15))
 (segment (start 110.331216 102.257626) (end 111.000117 102.926527) (width 0.25) (layer B.Cu) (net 15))
 (segment (start 147.699815 102.926527) (end 148.431216 102.195126) (width 0.25) (layer B.Cu) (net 15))
 (segment (start 130.050117 102.926527) (end 147.699815 102.926527) (width 0.25) (layer B.Cu) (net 15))
 (segment (start 129.381216 102.257626) (end 130.050117 102.926527) (width 0.25) (layer B.Cu) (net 15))
 (segment (start 166.749815 102.926527) (end 167.481216 102.195126) (width 0.25) (layer B.Cu) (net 15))
 (segment (start 149.162617 102.926527) (end 166.749815 102.926527) (width 0.25) (layer B.Cu) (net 15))
 (segment (start 148.431216 102.195126) (end 149.162617 102.926527) (width 0.25) (layer B.Cu) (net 15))
 (segment (start 110.331216 102.257626) (end 110.331216 103.981104) (width 0.25) (layer B.Cu) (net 15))
 (segment (start 110.331216 103.981104) (end 106.560848 107.751472) (width 0.25) (layer B.Cu) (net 15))
 (segment (start 106.560848 107.751472) (end 98.821792 107.751472) (width 0.25) (layer B.Cu) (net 15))
 (segment (start 94.349902 57.967774) (end 98.448992 53.868684) (width 0.25) (layer B.Cu) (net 15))
 (segment (start 94.349902 103.279582) (end 94.349902 57.967774) (width 0.25) (layer B.Cu) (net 15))
 (segment (start 98.821792 107.751472) (end 94.349902 103.279582) (width 0.25) (layer B.Cu) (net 15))
 (segment (start 126.471316 53.868684) (end 130.65125 49.68875) (width 0.25) (layer B.Cu) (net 15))
 (segment (start 98.448992 53.868684) (end 126.471316 53.868684) (width 0.25) (layer B.Cu) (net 15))
 (segment (start 125.951216 95.527626) (end 129.381216 98.957626) (width 0.25) (layer B.Cu) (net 31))
 (segment (start 123.983716 95.527626) (end 125.951216 95.527626) (width 0.25) (layer B.Cu) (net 31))
 (segment (start 145.063716 95.527626) (end 148.431216 98.895126) (width 0.25) (layer B.Cu) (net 30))
 (segment (start 143.033716 95.527626) (end 145.063716 95.527626) (width 0.25) (layer B.Cu) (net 30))
 (segment (start 164.113716 95.527626) (end 167.481216 98.895126) (width 0.25) (layer B.Cu) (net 29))
 (segment (start 162.083716 95.527626) (end 164.113716 95.527626) (width 0.25) (layer B.Cu) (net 29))
 (segment (start 106.901216 114.577626) (end 110.331216 118.007626) (width 0.25) (layer B.Cu) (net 28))
 (segment (start 104.933716 114.577626) (end 106.901216 114.577626) (width 0.25) (layer B.Cu) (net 28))
 (segment (start 111.000117 121.976527) (end 128.712315 121.976527) (width 0.25) (layer B.Cu) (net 2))
 (segment (start 128.712315 121.976527) (end 129.381216 121.307626) (width 0.25) (layer B.Cu) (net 2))
 (segment (start 110.331216 121.307626) (end 111.000117 121.976527) (width 0.25) (layer B.Cu) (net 2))
 (segment (start 130.050117 121.976527) (end 147.762315 121.976527) (width 0.25) (layer B.Cu) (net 2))
 (segment (start 147.762315 121.976527) (end 148.431216 121.307626) (width 0.25) (layer B.Cu) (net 2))
 (segment (start 129.381216 121.307626) (end 130.050117 121.976527) (width 0.25) (layer B.Cu) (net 2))
 (segment (start 166.812315 121.976527) (end 167.481216 121.307626) (width 0.25) (layer B.Cu) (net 2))
 (segment (start 149.100117 121.976527) (end 166.812315 121.976527) (width 0.25) (layer B.Cu) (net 2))
 (segment (start 148.431216 121.307626) (end 149.100117 121.976527) (width 0.25) (layer B.Cu) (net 2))
 (segment (start 98.262592 53.418674) (end 124.381326 53.418674) (width 0.25) (layer B.Cu) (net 2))
 (segment (start 93.899893 57.781373) (end 98.262592 53.418674) (width 0.25) (layer B.Cu) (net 2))
 (segment (start 124.381326 53.418674) (end 128.11125 49.68875) (width 0.25) (layer B.Cu) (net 2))
 (segment (start 93.899893 123.665493) (end 93.899893 57.781373) (width 0.25) (layer B.Cu) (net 2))
 (segment (start 97.035856 126.801456) (end 93.899893 123.665493) (width 0.25) (layer B.Cu) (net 2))
 (segment (start 106.560848 126.801456) (end 97.035856 126.801456) (width 0.25) (layer B.Cu) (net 2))
 (segment (start 110.331216 123.031088) (end 106.560848 126.801456) (width 0.25) (layer B.Cu) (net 2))
 (segment (start 110.331216 121.307626) (end 110.331216 123.031088) (width 0.25) (layer B.Cu) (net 2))
 (segment (start 125.951216 114.577626) (end 129.381216 118.007626) (width 0.25) (layer B.Cu) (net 27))
 (segment (start 123.983716 114.577626) (end 125.951216 114.577626) (width 0.25) (layer B.Cu) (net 27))
 (segment (start 145.001216 114.577626) (end 148.431216 118.007626) (width 0.25) (layer B.Cu) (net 26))
 (segment (start 143.033716 114.577626) (end 145.001216 114.577626) (width 0.25) (layer B.Cu) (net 26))
 (segment (start 164.051216 114.577626) (end 167.481216 118.007626) (width 0.25) (layer B.Cu) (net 1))
 (segment (start 162.083716 114.577626) (end 164.051216 114.577626) (width 0.25) (layer B.Cu) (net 1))
 (segment (start 98.583716 59.967626) (end 98.583716 117.117626) (width 0.25) (layer F.Cu) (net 18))
 (segment (start 132.595984 55.364016) (end 138.27125 49.68875) (width 0.25) (layer F.Cu) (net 18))
 (segment (start 101.20304 55.364016) (end 132.595984 55.364016) (width 0.25) (layer F.Cu) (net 18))
 (segment (start 98.583716 57.98334) (end 101.20304 55.364016) (width 0.25) (layer F.Cu) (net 18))
 (segment (start 98.583716 59.967626) (end 98.583716 57.98334) (width 0.25) (layer F.Cu) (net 18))
 (segment (start 117.633716 100.2296) (end 117.633716 117.117626) (width 0.25) (layer F.Cu) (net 19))
 (segment (start 117.633716 59.967626) (end 117.633716 100.2296) (width 0.25) (layer F.Cu) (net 19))
 (segment (start 117.633716 59.967626) (end 117.633716 57.983324) (width 0.25) (layer F.Cu) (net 19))
 (segment (start 134.685974 55.814026) (end 140.81125 49.68875) (width 0.25) (layer F.Cu) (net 19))
 (segment (start 119.803014 55.814026) (end 134.685974 55.814026) (width 0.25) (layer F.Cu) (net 19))
 (segment (start 117.633716 57.983324) (end 119.803014 55.814026) (width 0.25) (layer F.Cu) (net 19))
 (segment (start 136.683716 59.967626) (end 136.683716 117.117626) (width 0.25) (layer F.Cu) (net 20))
 (segment (start 136.683716 56.356284) (end 143.35125 49.68875) (width 0.25) (layer F.Cu) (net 20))
 (segment (start 136.683716 59.967626) (end 136.683716 56.356284) (width 0.25) (layer F.Cu) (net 20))
 (segment (start 155.733716 59.967626) (end 155.733716 117.117626) (width 0.25) (layer F.Cu) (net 21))
 (segment (start 145.89125 50.12516) (end 145.89125 49.68875) (width 0.25) (layer F.Cu) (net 21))
 (segment (start 155.733716 59.967626) (end 145.89125 50.12516) (width 0.25) (layer F.Cu) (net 21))
 (segment (start 116.70625 43.96875) (end 123.00625 43.96875) (width 0.25) (layer B.Cu) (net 4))
 (segment (start 143.99125 43.96875) (end 153.51125 34.44875) (width 0.25) (layer B.Cu) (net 4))
 (segment (start 123.00625 43.96875) (end 143.99125 43.96875) (width 0.25) (layer B.Cu) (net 4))
 (segment (start 116.70625 40.16875) (end 123.00625 40.16875) (width 0.25) (layer B.Cu) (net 5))
 (segment (start 145.25125 40.16875) (end 150.97125 34.44875) (width 0.25) (layer B.Cu) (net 5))
 (segment (start 123.00625 40.16875) (end 145.25125 40.16875) (width 0.25) (layer B.Cu) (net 5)))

